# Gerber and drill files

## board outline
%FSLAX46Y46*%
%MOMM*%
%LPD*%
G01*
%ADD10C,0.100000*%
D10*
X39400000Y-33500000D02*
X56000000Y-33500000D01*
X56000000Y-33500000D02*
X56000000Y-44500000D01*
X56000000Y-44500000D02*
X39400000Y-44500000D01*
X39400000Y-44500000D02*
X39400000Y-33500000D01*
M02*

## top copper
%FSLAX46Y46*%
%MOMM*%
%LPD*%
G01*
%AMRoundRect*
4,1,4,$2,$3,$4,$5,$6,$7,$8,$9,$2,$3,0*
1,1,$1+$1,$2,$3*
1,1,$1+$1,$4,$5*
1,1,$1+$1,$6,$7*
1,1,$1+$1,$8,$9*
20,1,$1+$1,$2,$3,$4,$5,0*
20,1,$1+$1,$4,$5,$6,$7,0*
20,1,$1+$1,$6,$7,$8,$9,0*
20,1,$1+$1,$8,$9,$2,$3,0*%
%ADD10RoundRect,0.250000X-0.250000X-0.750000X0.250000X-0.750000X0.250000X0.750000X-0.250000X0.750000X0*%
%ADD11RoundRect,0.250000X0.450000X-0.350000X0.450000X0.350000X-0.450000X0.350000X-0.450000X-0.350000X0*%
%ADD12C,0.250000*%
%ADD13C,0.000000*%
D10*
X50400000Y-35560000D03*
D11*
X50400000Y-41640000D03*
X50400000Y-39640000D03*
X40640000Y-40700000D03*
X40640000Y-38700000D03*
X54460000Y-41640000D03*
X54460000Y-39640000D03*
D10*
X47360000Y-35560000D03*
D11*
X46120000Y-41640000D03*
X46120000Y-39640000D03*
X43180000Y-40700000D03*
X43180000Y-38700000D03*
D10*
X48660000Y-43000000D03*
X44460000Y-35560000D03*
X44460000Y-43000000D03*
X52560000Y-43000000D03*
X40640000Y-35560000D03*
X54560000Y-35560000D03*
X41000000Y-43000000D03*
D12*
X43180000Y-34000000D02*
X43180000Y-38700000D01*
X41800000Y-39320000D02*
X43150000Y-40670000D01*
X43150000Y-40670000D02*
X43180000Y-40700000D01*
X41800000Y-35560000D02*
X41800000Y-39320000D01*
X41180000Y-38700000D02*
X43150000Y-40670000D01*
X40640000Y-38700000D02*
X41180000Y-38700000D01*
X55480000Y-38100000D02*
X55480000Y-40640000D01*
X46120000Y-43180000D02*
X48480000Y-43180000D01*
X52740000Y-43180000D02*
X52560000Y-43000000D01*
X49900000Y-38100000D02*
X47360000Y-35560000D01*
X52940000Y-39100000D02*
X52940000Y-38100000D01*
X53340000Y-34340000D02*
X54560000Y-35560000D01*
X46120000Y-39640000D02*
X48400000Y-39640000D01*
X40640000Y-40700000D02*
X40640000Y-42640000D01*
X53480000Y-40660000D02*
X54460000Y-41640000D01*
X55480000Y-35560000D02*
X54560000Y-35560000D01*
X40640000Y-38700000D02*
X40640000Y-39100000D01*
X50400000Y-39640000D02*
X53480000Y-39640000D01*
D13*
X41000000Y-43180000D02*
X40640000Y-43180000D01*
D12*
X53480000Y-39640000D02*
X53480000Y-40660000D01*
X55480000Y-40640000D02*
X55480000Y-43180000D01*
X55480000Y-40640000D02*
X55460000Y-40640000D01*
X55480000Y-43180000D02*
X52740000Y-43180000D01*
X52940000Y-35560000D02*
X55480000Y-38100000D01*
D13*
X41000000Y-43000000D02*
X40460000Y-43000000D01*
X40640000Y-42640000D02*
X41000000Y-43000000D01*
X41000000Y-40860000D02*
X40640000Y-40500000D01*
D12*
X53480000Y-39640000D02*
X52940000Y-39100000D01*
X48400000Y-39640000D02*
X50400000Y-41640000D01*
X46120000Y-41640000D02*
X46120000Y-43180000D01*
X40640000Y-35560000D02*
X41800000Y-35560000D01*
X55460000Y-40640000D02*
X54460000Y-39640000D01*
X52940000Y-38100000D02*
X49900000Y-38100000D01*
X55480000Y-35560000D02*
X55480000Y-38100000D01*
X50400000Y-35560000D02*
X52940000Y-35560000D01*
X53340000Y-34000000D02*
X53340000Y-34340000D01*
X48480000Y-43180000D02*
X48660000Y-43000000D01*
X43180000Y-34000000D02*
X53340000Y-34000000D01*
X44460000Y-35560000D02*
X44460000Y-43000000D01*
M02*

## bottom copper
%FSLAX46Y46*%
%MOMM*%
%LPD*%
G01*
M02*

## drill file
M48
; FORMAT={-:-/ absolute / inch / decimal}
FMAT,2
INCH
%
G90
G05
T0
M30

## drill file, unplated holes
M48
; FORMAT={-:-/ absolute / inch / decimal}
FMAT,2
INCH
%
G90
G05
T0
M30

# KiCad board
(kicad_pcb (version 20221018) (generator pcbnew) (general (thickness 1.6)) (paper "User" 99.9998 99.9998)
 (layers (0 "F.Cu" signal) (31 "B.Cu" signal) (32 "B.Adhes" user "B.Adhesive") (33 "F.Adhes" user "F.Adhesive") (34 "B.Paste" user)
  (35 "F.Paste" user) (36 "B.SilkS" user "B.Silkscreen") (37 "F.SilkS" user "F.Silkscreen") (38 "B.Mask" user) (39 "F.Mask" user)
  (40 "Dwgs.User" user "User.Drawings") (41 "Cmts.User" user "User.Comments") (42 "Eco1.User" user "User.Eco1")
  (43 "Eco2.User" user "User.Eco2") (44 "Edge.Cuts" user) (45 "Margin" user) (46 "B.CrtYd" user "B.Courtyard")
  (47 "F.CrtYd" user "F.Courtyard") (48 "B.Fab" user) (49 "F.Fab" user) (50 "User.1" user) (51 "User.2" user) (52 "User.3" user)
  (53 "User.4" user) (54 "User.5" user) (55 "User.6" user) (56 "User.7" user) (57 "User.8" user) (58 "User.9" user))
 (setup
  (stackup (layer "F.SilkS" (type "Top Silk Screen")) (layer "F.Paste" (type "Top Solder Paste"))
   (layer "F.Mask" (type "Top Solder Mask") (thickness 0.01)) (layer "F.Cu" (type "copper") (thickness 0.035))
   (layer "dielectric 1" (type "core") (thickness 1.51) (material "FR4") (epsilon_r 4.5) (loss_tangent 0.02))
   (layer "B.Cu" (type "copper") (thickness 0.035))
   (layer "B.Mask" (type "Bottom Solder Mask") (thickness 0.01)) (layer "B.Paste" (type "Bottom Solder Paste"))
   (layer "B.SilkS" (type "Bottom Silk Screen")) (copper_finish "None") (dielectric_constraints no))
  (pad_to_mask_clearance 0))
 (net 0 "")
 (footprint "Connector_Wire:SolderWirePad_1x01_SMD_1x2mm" (layer "F.Cu") (at 50.4 35.56)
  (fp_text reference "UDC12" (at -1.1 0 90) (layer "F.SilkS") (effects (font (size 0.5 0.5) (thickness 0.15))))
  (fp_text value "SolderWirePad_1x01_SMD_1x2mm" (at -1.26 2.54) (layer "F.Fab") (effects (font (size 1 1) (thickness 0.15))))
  (pad "1" smd roundrect (at 0 0) (size 1 2) (layers "F.Cu" "F.Paste" "F.Mask") (roundrect_rratio 0.25)))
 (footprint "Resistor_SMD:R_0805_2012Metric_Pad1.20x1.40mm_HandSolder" (layer "F.Cu") (at 50.4 40.64 90)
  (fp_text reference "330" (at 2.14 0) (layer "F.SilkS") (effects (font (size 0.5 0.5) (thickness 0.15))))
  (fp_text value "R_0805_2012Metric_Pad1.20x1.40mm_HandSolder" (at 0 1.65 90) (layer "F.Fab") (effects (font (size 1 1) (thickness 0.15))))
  (pad "1" smd roundrect (at -1 0 90) (size 1.2 1.4) (layers "F.Cu" "F.Paste" "F.Mask") (roundrect_rratio 0.2083333333))
  (pad "2" smd roundrect (at 1 0 90) (size 1.2 1.4) (layers "F.Cu" "F.Paste" "F.Mask") (roundrect_rratio 0.2083333333)))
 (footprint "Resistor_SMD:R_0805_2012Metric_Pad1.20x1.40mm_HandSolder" (layer "F.Cu") (at 40.64 39.7 90)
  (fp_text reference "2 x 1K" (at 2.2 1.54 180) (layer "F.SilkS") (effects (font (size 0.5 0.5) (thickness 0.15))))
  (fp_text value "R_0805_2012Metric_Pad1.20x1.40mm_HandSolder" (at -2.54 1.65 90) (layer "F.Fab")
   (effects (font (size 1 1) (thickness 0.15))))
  (pad "1" smd roundrect (at -1 0 90) (size 1.2 1.4) (layers "F.Cu" "F.Paste" "F.Mask") (roundrect_rratio 0.2083333333))
  (pad "2" smd roundrect (at 1 0 90) (size 1.2 1.4) (layers "F.Cu" "F.Paste" "F.Mask") (roundrect_rratio 0.2083333333)))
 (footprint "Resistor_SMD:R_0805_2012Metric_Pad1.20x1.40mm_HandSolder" (layer "F.Cu") (at 54.46 40.64 90)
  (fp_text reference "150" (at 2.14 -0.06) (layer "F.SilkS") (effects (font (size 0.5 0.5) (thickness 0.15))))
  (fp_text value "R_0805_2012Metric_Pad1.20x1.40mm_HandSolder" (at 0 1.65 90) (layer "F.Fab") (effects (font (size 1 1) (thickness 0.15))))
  (pad "1" smd roundrect (at -1 0 90) (size 1.2 1.4) (layers "F.Cu" "F.Paste" "F.Mask") (roundrect_rratio 0.2083333333))
  (pad "2" smd roundrect (at 1 0 90) (size 1.2 1.4) (layers "F.Cu" "F.Paste" "F.Mask") (roundrect_rratio 0.2083333333)))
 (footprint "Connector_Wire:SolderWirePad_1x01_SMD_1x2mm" (layer "F.Cu") (at 47.36 35.56)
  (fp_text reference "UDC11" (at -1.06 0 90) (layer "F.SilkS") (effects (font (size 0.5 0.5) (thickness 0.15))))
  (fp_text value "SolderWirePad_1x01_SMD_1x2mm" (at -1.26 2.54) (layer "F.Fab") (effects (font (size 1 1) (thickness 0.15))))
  (pad "1" smd roundrect (at 0 0) (size 1 2) (layers "F.Cu" "F.Paste" "F.Mask") (roundrect_rratio 0.25)))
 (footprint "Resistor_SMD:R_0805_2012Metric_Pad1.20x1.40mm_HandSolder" (layer "F.Cu") (at 46.12 40.64 90)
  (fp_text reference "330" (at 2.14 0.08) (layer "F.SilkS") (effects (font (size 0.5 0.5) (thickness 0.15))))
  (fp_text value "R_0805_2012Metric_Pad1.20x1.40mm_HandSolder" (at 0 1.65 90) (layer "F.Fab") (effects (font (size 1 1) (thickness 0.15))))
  (pad "1" smd roundrect (at -1 0 90) (size 1.2 1.4) (layers "F.Cu" "F.Paste" "F.Mask") (roundrect_rratio 0.2083333333))
  (pad "2" smd roundrect (at 1 0 90) (size 1.2 1.4) (layers "F.Cu" "F.Paste" "F.Mask") (roundrect_rratio 0.2083333333)))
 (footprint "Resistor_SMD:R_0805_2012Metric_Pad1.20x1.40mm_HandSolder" (layer "F.Cu") (at 43.18 39.7 90)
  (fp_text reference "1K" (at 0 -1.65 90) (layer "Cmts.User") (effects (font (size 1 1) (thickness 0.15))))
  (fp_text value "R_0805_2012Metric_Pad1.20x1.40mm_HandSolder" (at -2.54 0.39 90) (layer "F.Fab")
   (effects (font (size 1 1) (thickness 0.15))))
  (pad "1" smd roundrect (at -1 0 90) (size 1.2 1.4) (layers "F.Cu" "F.Paste" "F.Mask") (roundrect_rratio 0.2083333333))
  (pad "2" smd roundrect (at 1 0 90) (size 1.2 1.4) (layers "F.Cu" "F.Paste" "F.Mask") (roundrect_rratio 0.2083333333)))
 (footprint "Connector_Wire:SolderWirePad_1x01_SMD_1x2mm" (layer "F.Cu") (at 48.66 43)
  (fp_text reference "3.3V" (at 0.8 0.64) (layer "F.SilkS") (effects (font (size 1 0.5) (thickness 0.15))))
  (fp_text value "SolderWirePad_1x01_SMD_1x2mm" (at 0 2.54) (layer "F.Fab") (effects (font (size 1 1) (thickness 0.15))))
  (pad "1" smd roundrect (at 0 0) (size 1 2) (layers "F.Cu" "F.Paste" "F.Mask") (roundrect_rratio 0.25)))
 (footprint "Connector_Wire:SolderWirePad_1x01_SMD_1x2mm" (layer "F.Cu") (at 44.46 35.56)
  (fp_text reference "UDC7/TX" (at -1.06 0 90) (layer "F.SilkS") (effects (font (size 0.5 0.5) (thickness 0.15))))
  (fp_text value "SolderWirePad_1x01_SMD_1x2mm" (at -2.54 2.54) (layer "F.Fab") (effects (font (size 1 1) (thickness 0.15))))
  (pad "1" smd roundrect (at 0 0) (size 1 2) (layers "F.Cu" "F.Paste" "F.Mask") (roundrect_rratio 0.25)))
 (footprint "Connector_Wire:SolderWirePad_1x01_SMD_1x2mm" (layer "F.Cu") (at 44.46 43)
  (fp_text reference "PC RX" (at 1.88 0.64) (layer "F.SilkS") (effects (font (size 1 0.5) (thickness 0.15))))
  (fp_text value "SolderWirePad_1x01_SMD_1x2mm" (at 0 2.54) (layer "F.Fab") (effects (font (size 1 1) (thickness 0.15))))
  (pad "1" smd roundrect (at 0 0) (size 1 2) (layers "F.Cu" "F.Paste" "F.Mask") (roundrect_rratio 0.25)))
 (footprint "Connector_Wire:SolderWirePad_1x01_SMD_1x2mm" (layer "F.Cu") (at 52.56 43)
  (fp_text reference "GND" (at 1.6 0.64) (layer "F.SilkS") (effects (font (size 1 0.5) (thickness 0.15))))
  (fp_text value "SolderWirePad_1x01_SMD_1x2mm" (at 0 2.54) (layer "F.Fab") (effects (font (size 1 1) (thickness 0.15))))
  (pad "1" smd roundrect (at 0 0) (size 1 2) (layers "F.Cu" "F.Paste" "F.Mask") (roundrect_rratio 0.25)))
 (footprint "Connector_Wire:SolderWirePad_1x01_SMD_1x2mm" (layer "F.Cu") (at 40.64 35.56)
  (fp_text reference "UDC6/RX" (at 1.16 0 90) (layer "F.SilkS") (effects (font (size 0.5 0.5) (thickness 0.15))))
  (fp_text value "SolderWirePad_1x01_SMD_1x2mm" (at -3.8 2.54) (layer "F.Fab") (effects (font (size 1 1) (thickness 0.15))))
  (pad "1" smd roundrect (at 0 0) (size 1 2) (layers "F.Cu" "F.Paste" "F.Mask") (roundrect_rratio 0.25)))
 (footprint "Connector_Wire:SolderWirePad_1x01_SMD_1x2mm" (layer "F.Cu") (at 54.56 35.56)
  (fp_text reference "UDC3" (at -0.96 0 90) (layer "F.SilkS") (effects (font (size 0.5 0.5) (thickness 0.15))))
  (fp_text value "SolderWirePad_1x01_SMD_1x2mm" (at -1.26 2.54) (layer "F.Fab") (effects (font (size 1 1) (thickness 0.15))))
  (pad "1" smd roundrect (at 0 0) (size 1 2) (layers "F.Cu" "F.Paste" "F.Mask") (roundrect_rratio 0.25)))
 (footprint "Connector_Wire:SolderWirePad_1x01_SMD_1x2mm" (layer "F.Cu") (at 41 43)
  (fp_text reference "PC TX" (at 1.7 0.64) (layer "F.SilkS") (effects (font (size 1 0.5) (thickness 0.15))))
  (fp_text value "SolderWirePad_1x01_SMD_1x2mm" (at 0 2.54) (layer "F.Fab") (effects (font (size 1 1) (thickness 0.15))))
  (pad "1" smd roundrect (at 0 0) (size 1 2) (layers "F.Cu" "F.Paste" "F.Mask") (roundrect_rratio 0.25)))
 (gr_rect (start 39.4 33.5) (end 56 44.5) (stroke (width 0.1) (type default)) (fill none) (layer "Edge.Cuts"))
 (segment (start 55.48 38.1) (end 55.48 40.64) (width 0.25) (layer "F.Cu") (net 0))
 (segment (start 46.12 43.18) (end 48.48 43.18) (width 0.25) (layer "F.Cu") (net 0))
 (segment (start 52.74 43.18) (end 52.56 43) (width 0.25) (layer "F.Cu") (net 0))
 (segment (start 49.9 38.1) (end 47.36 35.56) (width 0.25) (layer "F.Cu") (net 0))
 (segment (start 52.94 39.1) (end 52.94 38.1) (width 0.25) (layer "F.Cu") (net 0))
 (segment (start 53.34 34.34) (end 54.56 35.56) (width 0.25) (layer "F.Cu") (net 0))
 (segment (start 46.12 39.64) (end 48.4 39.64) (width 0.25) (layer "F.Cu") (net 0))
 (segment (start 40.64 40.7) (end 40.64 42.64) (width 0.25) (layer "F.Cu") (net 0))
 (segment (start 53.48 40.66) (end 54.46 41.64) (width 0.25) (layer "F.Cu") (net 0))
 (segment (start 55.48 35.56) (end 54.56 35.56) (width 0.25) (layer "F.Cu") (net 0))
 (segment (start 40.64 38.7) (end 40.64 39.1) (width 0.25) (layer "F.Cu") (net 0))
 (segment (start 50.4 39.64) (end 53.48 39.64) (width 0.25) (layer "F.Cu") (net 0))
 (segment (start 41 43.18) (end 40.64 43.18) (width 0) (layer "F.Cu") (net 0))
 (segment (start 41.8 35.56) (end 41.8 39.32) (width 0.25) (layer "F.Cu") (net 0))
 (segment (start 53.48 39.64) (end 53.48 40.66) (width 0.25) (layer "F.Cu") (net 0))
 (segment (start 55.48 40.64) (end 55.48 43.18) (width 0.25) (layer "F.Cu") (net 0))
 (segment (start 55.48 40.64) (end 55.46 40.64) (width 0.25) (layer "F.Cu") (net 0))
 (segment (start 55.48 43.18) (end 52.74 43.18) (width 0.25) (layer "F.Cu") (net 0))
 (segment (start 52.94 35.56) (end 55.48 38.1) (width 0.25) (layer "F.Cu") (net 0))
 (segment (start 41 43) (end 40.46 43) (width 0) (layer "F.Cu") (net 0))
 (segment (start 40.64 42.64) (end 41 43) (width 0) (layer "F.Cu") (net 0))
 (segment (start 41 40.86) (end 40.64 40.5) (width 0) (layer "F.Cu") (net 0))
 (segment (start 40.64 38.7) (end 41.18 38.7) (width 0.25) (layer "F.Cu") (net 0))
 (segment (start 53.48 39.64) (end 52.94 39.1) (width 0.25) (layer "F.Cu") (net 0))
 (segment (start 48.4 39.64) (end 50.4 41.64) (width 0.25) (layer "F.Cu") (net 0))
 (segment (start 41.8 39.32) (end 43.15 40.67) (width 0.25) (layer "F.Cu") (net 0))
 (segment (start 46.12 41.64) (end 46.12 43.18) (width 0.25) (layer "F.Cu") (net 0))
 (segment (start 40.64 35.56) (end 41.8 35.56) (width 0.25) (layer "F.Cu") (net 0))
 (segment (start 55.46 40.64) (end 54.46 39.64) (width 0.25) (layer "F.Cu") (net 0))
 (segment (start 52.94 38.1) (end 49.9 38.1) (width 0.25) (layer "F.Cu") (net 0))
 (segment (start 55.48 35.56) (end 55.48 38.1) (width 0.25) (layer "F.Cu") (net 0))
 (segment (start 50.4 35.56) (end 52.94 35.56) (width 0.25) (layer "F.Cu") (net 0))
 (segment (start 53.34 34) (end 53.34 34.34) (width 0.25) (layer "F.Cu") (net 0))
 (segment (start 48.48 43.18) (end 48.66 43) (width 0.25) (layer "F.Cu") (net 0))
 (segment (start 43.15 40.67) (end 43.18 40.7) (width 0.25) (layer "F.Cu") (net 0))
 (segment (start 43.18 34) (end 53.34 34) (width 0.25) (layer "F.Cu") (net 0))
 (segment (start 43.18 34) (end 43.18 38.7) (width 0.25) (layer "F.Cu") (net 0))
 (segment (start 41.18 38.7) (end 43.15 40.67) (width 0.25) (layer "F.Cu") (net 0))
 (segment (start 44.46 35.56) (end 44.46 43) (width 0.25) (layer "F.Cu") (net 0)))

